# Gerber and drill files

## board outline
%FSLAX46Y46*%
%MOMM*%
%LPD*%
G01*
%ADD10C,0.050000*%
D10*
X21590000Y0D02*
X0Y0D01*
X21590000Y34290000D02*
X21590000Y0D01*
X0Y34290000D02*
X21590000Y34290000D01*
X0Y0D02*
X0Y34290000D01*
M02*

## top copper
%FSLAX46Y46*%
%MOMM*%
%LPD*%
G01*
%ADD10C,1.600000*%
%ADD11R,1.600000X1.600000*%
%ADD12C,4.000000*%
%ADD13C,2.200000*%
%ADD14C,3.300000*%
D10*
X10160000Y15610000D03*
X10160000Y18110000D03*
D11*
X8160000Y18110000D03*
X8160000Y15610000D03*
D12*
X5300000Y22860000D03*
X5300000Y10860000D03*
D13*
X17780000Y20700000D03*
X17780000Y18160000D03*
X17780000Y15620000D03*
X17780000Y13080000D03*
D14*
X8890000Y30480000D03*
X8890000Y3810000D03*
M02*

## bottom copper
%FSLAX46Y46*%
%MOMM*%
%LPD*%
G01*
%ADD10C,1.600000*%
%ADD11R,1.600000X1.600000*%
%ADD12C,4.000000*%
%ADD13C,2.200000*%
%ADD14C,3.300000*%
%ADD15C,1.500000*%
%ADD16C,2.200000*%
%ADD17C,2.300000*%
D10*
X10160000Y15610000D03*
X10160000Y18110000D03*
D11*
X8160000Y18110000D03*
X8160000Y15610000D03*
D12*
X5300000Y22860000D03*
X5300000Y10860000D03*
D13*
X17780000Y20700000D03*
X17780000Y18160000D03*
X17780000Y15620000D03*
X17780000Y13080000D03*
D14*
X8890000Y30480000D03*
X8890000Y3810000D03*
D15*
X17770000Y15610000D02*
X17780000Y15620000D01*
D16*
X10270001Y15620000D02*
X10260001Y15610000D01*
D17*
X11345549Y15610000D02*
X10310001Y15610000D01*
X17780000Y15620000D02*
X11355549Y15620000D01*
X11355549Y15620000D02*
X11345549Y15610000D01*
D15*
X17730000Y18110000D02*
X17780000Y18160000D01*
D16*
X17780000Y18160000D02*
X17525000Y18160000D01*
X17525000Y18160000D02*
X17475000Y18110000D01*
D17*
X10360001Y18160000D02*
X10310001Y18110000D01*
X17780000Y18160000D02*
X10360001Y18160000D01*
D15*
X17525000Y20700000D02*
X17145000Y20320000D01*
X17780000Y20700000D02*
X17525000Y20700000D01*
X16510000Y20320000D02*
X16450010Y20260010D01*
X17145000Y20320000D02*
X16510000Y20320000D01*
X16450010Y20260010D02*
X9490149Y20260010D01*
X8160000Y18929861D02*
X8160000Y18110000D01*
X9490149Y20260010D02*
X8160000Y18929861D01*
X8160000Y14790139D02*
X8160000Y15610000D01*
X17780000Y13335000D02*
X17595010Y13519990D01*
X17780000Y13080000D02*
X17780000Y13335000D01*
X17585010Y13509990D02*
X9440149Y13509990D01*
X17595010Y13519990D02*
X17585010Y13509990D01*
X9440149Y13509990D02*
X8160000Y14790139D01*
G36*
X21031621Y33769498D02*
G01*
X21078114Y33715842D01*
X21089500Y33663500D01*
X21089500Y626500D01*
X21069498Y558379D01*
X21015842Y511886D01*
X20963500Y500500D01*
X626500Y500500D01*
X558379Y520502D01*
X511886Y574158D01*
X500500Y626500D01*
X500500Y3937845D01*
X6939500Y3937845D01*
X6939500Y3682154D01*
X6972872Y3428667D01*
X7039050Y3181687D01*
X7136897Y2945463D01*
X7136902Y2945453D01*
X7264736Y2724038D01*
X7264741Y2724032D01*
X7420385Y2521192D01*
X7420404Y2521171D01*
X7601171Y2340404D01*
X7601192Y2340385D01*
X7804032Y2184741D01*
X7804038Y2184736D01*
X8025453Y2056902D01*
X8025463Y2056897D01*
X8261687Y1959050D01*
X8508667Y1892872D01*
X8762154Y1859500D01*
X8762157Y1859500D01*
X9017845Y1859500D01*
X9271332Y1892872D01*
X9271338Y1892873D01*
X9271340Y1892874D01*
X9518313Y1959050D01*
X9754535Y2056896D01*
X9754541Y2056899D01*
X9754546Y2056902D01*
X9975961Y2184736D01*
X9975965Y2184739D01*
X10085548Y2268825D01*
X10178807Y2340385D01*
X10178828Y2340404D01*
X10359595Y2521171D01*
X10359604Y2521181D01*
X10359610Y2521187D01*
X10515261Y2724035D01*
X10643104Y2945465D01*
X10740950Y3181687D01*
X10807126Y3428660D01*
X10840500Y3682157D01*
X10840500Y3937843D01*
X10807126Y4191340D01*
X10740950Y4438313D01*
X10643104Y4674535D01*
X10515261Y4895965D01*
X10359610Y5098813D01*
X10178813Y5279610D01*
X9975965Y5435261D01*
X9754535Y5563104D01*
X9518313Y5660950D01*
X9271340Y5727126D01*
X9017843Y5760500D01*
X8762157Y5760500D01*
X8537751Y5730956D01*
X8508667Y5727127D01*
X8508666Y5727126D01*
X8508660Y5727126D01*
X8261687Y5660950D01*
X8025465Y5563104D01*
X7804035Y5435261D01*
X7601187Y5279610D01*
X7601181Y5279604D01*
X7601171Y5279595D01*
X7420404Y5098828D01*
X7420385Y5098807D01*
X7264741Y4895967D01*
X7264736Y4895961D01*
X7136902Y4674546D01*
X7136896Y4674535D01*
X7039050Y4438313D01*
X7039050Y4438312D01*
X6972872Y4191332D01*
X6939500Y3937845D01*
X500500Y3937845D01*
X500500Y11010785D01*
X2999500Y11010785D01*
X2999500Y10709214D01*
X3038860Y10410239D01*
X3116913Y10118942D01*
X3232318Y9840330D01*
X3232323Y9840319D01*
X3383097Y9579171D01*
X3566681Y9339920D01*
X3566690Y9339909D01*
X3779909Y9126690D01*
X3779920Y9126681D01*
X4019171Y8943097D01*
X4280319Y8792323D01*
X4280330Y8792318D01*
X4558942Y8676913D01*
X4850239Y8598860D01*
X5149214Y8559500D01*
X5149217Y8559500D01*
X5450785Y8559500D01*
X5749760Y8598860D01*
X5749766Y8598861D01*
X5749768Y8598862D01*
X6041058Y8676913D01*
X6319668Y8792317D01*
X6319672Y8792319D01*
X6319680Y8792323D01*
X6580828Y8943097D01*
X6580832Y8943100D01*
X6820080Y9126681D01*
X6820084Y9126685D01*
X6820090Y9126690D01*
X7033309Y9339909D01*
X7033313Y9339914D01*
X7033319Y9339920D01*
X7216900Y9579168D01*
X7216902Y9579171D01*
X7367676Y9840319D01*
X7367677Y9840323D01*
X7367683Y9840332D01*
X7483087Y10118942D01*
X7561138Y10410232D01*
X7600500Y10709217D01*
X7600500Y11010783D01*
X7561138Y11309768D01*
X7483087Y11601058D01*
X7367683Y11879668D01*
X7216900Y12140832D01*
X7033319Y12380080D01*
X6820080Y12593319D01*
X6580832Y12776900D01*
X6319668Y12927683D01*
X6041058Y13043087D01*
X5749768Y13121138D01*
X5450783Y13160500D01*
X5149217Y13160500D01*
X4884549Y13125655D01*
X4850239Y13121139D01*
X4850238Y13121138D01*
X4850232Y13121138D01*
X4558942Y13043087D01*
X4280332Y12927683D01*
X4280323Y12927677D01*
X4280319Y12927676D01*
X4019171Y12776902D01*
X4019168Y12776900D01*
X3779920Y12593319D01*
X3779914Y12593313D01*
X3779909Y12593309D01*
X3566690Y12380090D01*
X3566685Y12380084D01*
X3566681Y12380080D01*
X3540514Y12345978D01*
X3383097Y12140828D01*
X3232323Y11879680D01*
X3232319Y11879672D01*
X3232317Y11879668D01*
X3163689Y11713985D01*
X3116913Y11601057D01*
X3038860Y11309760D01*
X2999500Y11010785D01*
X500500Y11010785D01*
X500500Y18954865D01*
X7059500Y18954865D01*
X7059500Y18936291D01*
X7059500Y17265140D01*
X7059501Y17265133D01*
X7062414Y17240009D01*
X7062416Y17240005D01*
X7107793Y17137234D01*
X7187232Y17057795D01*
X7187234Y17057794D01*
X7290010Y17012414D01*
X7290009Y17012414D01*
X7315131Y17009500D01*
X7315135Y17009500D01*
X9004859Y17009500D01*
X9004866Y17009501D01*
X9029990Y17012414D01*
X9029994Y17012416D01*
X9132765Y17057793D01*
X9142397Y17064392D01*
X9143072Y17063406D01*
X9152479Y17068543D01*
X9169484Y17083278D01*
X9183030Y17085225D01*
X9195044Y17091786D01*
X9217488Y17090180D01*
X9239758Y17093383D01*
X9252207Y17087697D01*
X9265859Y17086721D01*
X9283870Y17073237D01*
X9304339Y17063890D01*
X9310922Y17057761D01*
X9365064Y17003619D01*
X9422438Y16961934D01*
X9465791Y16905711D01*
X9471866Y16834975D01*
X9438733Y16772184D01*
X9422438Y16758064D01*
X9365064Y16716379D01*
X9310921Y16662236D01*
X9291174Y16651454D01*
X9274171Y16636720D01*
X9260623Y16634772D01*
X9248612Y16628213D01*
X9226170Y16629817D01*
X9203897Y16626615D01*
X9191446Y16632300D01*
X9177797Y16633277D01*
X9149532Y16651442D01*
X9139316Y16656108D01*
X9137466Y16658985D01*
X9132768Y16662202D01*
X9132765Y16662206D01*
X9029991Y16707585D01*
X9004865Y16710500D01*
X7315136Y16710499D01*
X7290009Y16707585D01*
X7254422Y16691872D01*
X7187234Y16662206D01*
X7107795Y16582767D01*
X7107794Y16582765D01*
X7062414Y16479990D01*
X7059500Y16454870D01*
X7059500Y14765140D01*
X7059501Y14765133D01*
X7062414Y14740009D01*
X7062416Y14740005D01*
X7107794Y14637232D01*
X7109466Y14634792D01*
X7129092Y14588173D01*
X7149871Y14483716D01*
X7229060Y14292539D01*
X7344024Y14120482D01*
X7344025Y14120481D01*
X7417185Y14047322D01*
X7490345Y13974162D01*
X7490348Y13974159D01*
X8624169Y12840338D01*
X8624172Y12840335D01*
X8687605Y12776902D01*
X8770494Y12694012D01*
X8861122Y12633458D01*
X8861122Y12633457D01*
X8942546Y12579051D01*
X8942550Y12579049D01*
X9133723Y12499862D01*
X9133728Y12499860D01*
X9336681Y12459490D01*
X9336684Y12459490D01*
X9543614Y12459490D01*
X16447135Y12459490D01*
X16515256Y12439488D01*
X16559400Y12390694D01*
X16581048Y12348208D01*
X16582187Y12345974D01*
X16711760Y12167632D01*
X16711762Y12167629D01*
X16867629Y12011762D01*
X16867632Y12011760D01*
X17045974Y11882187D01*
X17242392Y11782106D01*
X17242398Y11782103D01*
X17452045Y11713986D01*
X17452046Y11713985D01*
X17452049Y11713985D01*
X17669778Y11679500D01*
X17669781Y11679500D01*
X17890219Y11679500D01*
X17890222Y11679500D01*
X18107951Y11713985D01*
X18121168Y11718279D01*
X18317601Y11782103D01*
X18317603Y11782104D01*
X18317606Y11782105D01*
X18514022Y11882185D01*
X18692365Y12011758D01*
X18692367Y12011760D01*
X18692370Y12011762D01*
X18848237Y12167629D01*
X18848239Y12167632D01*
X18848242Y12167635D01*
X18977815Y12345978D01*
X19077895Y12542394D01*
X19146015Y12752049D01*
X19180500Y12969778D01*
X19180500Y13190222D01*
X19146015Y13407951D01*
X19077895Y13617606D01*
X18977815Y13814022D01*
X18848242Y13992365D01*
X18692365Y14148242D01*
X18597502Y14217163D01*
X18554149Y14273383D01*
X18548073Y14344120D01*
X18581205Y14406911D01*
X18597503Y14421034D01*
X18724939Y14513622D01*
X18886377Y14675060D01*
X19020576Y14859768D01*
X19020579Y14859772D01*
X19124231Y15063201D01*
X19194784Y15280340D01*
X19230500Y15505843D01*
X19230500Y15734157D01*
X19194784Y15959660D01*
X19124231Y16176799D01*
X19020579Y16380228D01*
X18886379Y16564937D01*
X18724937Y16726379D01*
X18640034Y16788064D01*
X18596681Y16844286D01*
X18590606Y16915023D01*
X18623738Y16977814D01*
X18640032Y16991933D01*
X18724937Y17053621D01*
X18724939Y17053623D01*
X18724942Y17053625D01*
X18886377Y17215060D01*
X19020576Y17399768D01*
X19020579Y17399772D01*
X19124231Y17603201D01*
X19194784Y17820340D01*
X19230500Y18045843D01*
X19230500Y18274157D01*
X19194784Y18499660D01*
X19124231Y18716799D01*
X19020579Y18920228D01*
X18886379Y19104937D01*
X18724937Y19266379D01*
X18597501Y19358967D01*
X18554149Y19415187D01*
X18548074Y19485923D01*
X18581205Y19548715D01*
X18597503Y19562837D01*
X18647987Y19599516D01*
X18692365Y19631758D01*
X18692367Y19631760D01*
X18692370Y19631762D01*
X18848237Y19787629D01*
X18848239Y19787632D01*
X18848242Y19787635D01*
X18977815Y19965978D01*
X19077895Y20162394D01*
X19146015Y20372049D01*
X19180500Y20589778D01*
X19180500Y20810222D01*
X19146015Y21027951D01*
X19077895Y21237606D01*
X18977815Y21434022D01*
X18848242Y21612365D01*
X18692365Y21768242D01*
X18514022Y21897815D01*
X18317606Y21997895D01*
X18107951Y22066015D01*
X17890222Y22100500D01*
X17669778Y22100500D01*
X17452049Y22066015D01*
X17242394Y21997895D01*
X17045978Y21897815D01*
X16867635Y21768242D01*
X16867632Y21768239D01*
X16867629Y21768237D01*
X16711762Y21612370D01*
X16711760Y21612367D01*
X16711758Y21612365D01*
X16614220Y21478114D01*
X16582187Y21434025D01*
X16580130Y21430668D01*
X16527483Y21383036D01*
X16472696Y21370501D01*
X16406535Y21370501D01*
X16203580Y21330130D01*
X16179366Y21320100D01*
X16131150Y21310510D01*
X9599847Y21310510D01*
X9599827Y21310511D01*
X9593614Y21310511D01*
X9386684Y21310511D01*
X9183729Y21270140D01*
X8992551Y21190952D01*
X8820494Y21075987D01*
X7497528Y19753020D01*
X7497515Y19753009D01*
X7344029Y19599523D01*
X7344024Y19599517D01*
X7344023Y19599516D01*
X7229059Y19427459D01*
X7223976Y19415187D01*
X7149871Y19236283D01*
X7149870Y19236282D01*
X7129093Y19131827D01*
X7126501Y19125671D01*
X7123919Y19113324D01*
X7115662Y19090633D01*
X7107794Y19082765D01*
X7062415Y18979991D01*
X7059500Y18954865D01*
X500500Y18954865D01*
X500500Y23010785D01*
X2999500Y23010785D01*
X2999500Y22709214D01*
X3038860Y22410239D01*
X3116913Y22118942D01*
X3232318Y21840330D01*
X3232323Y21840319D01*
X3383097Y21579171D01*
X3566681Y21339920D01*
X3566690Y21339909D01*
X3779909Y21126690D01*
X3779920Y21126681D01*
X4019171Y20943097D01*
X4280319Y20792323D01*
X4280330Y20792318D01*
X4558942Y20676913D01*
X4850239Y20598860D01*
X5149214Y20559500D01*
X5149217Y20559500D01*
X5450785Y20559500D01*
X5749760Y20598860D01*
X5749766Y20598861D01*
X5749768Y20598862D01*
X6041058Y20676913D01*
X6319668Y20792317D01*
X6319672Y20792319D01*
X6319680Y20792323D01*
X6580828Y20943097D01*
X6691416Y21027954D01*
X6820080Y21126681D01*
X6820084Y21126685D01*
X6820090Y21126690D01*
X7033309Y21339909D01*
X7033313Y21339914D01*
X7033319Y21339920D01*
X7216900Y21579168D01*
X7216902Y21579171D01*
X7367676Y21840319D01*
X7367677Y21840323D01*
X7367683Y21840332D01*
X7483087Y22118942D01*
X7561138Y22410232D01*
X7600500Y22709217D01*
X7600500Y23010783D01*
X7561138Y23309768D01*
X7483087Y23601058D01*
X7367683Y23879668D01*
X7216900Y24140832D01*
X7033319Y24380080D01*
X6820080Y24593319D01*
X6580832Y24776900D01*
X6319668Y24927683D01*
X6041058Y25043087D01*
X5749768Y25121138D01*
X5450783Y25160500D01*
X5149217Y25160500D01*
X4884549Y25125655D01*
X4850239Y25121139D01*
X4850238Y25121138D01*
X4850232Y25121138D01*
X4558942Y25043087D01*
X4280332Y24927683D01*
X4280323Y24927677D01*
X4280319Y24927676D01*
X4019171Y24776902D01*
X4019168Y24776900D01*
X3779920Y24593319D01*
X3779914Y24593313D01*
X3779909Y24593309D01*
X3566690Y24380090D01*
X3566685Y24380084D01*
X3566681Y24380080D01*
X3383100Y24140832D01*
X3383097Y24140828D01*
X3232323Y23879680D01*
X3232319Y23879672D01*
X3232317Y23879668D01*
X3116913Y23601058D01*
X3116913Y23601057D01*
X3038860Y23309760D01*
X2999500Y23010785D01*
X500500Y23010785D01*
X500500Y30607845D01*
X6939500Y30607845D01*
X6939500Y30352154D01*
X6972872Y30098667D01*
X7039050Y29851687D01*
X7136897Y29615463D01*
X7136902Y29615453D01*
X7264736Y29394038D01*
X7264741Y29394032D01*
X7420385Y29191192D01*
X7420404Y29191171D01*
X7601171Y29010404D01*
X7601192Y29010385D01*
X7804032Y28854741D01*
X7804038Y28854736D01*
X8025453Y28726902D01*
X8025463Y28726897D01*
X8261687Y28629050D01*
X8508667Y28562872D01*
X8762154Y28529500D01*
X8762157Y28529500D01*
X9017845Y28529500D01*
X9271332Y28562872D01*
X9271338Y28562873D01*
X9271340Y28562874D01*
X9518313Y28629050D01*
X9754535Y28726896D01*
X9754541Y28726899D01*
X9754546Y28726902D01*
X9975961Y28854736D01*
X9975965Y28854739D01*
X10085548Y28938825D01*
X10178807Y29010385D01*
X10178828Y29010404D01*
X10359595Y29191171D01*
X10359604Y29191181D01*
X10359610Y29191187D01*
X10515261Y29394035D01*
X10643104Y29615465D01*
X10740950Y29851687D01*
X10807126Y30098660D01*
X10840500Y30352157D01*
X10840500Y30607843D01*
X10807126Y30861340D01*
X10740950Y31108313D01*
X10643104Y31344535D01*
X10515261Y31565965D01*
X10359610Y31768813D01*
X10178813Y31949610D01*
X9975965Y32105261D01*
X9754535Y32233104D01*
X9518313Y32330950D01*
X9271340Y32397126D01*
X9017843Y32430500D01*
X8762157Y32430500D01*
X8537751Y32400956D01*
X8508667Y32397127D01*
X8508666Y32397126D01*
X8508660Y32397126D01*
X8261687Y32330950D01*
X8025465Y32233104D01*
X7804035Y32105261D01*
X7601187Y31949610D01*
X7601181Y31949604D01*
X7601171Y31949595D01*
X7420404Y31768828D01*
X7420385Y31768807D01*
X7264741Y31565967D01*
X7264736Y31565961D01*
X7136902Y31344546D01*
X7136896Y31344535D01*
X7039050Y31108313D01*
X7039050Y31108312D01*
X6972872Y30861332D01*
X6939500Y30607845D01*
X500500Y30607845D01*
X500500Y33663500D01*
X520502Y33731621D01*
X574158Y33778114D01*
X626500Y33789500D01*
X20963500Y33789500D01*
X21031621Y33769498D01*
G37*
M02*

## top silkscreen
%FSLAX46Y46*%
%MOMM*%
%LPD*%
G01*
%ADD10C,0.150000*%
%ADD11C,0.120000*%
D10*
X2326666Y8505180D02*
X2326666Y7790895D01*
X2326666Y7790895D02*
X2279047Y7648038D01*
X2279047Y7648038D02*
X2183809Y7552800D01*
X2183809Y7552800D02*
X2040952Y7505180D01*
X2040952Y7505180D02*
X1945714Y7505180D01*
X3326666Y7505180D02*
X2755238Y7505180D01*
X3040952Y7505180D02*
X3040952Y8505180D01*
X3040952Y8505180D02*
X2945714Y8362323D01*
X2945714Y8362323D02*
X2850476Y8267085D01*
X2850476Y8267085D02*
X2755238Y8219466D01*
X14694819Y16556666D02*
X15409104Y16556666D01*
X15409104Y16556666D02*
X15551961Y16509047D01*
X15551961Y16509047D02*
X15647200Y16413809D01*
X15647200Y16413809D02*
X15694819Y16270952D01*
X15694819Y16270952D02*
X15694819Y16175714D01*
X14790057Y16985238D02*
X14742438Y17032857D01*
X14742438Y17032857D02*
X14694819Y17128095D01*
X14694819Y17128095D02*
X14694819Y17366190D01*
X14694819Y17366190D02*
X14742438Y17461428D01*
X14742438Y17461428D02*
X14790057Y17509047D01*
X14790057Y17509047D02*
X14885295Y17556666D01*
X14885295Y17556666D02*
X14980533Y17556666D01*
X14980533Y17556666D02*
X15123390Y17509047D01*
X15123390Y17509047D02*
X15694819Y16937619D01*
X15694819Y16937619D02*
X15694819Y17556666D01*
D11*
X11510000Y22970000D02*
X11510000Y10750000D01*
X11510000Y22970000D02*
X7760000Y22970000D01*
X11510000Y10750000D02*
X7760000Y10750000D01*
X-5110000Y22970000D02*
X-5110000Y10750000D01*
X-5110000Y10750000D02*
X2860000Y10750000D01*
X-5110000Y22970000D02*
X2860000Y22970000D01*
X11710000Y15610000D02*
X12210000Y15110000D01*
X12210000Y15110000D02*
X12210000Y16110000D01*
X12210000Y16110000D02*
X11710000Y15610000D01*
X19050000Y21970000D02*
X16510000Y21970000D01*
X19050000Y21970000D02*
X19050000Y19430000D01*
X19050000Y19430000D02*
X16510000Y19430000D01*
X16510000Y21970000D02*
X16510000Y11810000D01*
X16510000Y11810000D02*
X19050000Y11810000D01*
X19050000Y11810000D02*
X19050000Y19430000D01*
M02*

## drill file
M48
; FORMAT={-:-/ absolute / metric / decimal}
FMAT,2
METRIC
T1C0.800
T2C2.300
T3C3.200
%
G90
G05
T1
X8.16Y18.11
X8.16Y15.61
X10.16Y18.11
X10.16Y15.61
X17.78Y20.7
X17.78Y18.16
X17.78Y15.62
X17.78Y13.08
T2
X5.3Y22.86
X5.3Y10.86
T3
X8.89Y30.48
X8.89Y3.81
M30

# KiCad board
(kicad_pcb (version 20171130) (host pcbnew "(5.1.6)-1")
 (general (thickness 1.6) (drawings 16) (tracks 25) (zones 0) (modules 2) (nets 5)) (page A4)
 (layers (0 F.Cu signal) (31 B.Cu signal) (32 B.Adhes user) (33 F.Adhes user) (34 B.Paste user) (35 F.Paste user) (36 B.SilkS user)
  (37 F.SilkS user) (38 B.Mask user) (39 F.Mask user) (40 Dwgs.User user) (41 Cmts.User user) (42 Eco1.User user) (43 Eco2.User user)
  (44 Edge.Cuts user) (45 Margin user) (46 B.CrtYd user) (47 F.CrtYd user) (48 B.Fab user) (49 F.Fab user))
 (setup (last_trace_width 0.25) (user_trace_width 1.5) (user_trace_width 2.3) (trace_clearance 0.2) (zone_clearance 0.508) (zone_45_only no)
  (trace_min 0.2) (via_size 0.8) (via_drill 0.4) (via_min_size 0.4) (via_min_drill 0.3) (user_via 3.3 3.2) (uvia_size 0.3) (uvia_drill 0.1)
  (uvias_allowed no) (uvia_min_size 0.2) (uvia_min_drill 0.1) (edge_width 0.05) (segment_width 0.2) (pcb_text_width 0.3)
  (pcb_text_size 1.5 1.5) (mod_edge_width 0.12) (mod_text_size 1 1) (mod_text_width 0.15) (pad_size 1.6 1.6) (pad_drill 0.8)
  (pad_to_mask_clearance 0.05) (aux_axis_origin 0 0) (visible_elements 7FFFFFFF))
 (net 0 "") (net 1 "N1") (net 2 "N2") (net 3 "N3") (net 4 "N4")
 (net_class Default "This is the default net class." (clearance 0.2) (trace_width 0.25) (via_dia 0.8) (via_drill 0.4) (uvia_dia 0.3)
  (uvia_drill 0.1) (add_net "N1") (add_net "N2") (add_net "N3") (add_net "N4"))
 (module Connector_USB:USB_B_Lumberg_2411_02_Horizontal (layer F.Cu) (at 10.16 -15.61 180)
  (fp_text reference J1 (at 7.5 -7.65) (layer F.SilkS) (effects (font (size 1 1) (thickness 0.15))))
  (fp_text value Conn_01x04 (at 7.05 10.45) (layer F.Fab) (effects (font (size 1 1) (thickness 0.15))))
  (fp_line (start -1.35 7.36) (end -1.35 -4.86) (layer F.SilkS) (width 0.12))
  (fp_line (start -1.35 7.36) (end 2.4 7.36) (layer F.SilkS) (width 0.12))
  (fp_line (start -1.35 -4.86) (end 2.4 -4.86) (layer F.SilkS) (width 0.12))
  (fp_line (start 15.27 7.36) (end 15.27 -4.86) (layer F.SilkS) (width 0.12))
  (fp_line (start 15.27 -4.86) (end 7.3 -4.86) (layer F.SilkS) (width 0.12))
  (fp_line (start 15.27 7.36) (end 7.3 7.36) (layer F.SilkS) (width 0.12))
  (fp_line (start -1.55 0) (end -2.05 -0.5) (layer F.SilkS) (width 0.12))
  (fp_line (start -2.05 -0.5) (end -2.05 0.5) (layer F.SilkS) (width 0.12))
  (fp_line (start -2.05 0.5) (end -1.55 0) (layer F.SilkS) (width 0.12))
  (pad 1 thru_hole circle (at 0 0 270) (size 1.6 1.6) (drill 0.8) (layers *.Cu *.Mask) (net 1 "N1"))
  (pad 2 thru_hole circle (at 0 2.5 270) (size 1.6 1.6) (drill 0.8) (layers *.Cu *.Mask) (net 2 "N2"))
  (pad 3 thru_hole rect (at 2 2.5 270) (size 1.6 1.6) (drill 0.8) (layers *.Cu *.Mask) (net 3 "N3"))
  (pad 4 thru_hole rect (at 2 0 270) (size 1.6 1.6) (drill 0.8) (layers *.Cu *.Mask) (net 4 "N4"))
  (pad 5 thru_hole circle (at 4.86 7.25 270) (size 4 4) (drill 2.3) (layers *.Cu *.Mask))
  (pad 5 thru_hole circle (at 4.86 -4.75 270) (size 4 4) (drill 2.3) (layers *.Cu *.Mask)))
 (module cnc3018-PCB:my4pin (layer F.Cu) (at 17.78 -20.7 270)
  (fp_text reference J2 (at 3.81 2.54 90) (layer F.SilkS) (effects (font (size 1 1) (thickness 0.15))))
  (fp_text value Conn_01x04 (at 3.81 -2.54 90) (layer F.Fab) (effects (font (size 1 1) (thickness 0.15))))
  (fp_line (start -1.27 -1.27) (end -1.27 1.27) (layer F.SilkS) (width 0.12))
  (fp_line (start -1.27 -1.27) (end 1.27 -1.27) (layer F.SilkS) (width 0.12))
  (fp_line (start 1.27 -1.27) (end 1.27 1.27) (layer F.SilkS) (width 0.12))
  (fp_line (start -1.27 1.27) (end 8.89 1.27) (layer F.SilkS) (width 0.12))
  (fp_line (start 8.89 1.27) (end 8.89 -1.27) (layer F.SilkS) (width 0.12))
  (fp_line (start 8.89 -1.27) (end 1.27 -1.27) (layer F.SilkS) (width 0.12))
  (pad 1 thru_hole circle (at 0 0 270) (size 2.2 2.2) (drill 0.8) (layers *.Cu *.Mask) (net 3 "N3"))
  (pad 2 thru_hole circle (at 2.54 0 270) (size 2.2 2.2) (drill 0.8) (layers *.Cu *.Mask) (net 2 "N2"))
  (pad 3 thru_hole circle (at 5.08 0 270) (size 2.2 2.2) (drill 0.8) (layers *.Cu *.Mask) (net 1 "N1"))
  (pad 4 thru_hole circle (at 7.62 0 270) (size 2.2 2.2) (drill 0.8) (layers *.Cu *.Mask) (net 4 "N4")))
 (gr_line (start 21.59 0) (end 0 0) (layer Edge.Cuts) (width 0.05))
 (gr_line (start 21.59 -34.29) (end 21.59 0) (layer Edge.Cuts) (width 0.05))
 (gr_line (start 0 -34.29) (end 21.59 -34.29) (layer Edge.Cuts) (width 0.05))
 (gr_line (start 0 0) (end 0 -34.29) (layer Edge.Cuts) (width 0.05))
 (via (at 8.89 -30.48) (size 3.3) (drill 3.2) (layers F.Cu B.Cu) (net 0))
 (via (at 8.89 -3.81) (size 3.3) (drill 3.2) (layers F.Cu B.Cu) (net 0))
 (segment (start 17.77 -15.61) (end 17.78 -15.62) (width 1.5) (layer B.Cu) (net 1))
 (segment (start 10.270001 -15.62) (end 10.260001 -15.61) (width 2.2) (layer B.Cu) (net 1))
 (segment (start 11.345549 -15.61) (end 10.310001 -15.61) (width 2.3) (layer B.Cu) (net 1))
 (segment (start 17.78 -15.62) (end 11.355549 -15.62) (width 2.3) (layer B.Cu) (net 1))
 (segment (start 11.355549 -15.62) (end 11.345549 -15.61) (width 2.3) (layer B.Cu) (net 1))
 (segment (start 17.73 -18.11) (end 17.78 -18.16) (width 1.5) (layer B.Cu) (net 2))
 (segment (start 17.78 -18.16) (end 17.525 -18.16) (width 2.2) (layer B.Cu) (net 2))
 (segment (start 17.525 -18.16) (end 17.475 -18.11) (width 2.2) (layer B.Cu) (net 2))
 (segment (start 10.360001 -18.16) (end 10.310001 -18.11) (width 2.3) (layer B.Cu) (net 2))
 (segment (start 17.78 -18.16) (end 10.360001 -18.16) (width 2.3) (layer B.Cu) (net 2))
 (segment (start 17.525 -20.7) (end 17.145 -20.32) (width 1.5) (layer B.Cu) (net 3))
 (segment (start 17.78 -20.7) (end 17.525 -20.7) (width 1.5) (layer B.Cu) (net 3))
 (segment (start 16.51 -20.32) (end 16.45001 -20.26001) (width 1.5) (layer B.Cu) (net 3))
 (segment (start 17.145 -20.32) (end 16.51 -20.32) (width 1.5) (layer B.Cu) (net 3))
 (segment (start 16.45001 -20.26001) (end 9.490149 -20.26001) (width 1.5) (layer B.Cu) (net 3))
 (segment (start 8.16 -18.929861) (end 8.16 -18.11) (width 1.5) (layer B.Cu) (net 3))
 (segment (start 9.490149 -20.26001) (end 8.16 -18.929861) (width 1.5) (layer B.Cu) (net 3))
 (segment (start 8.16 -14.790139) (end 8.16 -15.61) (width 1.5) (layer B.Cu) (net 4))
 (segment (start 17.78 -13.335) (end 17.59501 -13.51999) (width 1.5) (layer B.Cu) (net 4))
 (segment (start 17.78 -13.08) (end 17.78 -13.335) (width 1.5) (layer B.Cu) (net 4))
 (segment (start 17.58501 -13.50999) (end 9.440149 -13.50999) (width 1.5) (layer B.Cu) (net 4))
 (segment (start 17.59501 -13.51999) (end 17.58501 -13.50999) (width 1.5) (layer B.Cu) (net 4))
 (segment (start 9.440149 -13.50999) (end 8.16 -14.790139) (width 1.5) (layer B.Cu) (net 4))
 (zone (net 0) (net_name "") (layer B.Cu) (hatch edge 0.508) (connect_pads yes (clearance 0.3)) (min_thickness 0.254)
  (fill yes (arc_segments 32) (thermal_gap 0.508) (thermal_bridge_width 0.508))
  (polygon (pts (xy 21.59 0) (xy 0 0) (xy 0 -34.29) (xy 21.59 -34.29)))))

